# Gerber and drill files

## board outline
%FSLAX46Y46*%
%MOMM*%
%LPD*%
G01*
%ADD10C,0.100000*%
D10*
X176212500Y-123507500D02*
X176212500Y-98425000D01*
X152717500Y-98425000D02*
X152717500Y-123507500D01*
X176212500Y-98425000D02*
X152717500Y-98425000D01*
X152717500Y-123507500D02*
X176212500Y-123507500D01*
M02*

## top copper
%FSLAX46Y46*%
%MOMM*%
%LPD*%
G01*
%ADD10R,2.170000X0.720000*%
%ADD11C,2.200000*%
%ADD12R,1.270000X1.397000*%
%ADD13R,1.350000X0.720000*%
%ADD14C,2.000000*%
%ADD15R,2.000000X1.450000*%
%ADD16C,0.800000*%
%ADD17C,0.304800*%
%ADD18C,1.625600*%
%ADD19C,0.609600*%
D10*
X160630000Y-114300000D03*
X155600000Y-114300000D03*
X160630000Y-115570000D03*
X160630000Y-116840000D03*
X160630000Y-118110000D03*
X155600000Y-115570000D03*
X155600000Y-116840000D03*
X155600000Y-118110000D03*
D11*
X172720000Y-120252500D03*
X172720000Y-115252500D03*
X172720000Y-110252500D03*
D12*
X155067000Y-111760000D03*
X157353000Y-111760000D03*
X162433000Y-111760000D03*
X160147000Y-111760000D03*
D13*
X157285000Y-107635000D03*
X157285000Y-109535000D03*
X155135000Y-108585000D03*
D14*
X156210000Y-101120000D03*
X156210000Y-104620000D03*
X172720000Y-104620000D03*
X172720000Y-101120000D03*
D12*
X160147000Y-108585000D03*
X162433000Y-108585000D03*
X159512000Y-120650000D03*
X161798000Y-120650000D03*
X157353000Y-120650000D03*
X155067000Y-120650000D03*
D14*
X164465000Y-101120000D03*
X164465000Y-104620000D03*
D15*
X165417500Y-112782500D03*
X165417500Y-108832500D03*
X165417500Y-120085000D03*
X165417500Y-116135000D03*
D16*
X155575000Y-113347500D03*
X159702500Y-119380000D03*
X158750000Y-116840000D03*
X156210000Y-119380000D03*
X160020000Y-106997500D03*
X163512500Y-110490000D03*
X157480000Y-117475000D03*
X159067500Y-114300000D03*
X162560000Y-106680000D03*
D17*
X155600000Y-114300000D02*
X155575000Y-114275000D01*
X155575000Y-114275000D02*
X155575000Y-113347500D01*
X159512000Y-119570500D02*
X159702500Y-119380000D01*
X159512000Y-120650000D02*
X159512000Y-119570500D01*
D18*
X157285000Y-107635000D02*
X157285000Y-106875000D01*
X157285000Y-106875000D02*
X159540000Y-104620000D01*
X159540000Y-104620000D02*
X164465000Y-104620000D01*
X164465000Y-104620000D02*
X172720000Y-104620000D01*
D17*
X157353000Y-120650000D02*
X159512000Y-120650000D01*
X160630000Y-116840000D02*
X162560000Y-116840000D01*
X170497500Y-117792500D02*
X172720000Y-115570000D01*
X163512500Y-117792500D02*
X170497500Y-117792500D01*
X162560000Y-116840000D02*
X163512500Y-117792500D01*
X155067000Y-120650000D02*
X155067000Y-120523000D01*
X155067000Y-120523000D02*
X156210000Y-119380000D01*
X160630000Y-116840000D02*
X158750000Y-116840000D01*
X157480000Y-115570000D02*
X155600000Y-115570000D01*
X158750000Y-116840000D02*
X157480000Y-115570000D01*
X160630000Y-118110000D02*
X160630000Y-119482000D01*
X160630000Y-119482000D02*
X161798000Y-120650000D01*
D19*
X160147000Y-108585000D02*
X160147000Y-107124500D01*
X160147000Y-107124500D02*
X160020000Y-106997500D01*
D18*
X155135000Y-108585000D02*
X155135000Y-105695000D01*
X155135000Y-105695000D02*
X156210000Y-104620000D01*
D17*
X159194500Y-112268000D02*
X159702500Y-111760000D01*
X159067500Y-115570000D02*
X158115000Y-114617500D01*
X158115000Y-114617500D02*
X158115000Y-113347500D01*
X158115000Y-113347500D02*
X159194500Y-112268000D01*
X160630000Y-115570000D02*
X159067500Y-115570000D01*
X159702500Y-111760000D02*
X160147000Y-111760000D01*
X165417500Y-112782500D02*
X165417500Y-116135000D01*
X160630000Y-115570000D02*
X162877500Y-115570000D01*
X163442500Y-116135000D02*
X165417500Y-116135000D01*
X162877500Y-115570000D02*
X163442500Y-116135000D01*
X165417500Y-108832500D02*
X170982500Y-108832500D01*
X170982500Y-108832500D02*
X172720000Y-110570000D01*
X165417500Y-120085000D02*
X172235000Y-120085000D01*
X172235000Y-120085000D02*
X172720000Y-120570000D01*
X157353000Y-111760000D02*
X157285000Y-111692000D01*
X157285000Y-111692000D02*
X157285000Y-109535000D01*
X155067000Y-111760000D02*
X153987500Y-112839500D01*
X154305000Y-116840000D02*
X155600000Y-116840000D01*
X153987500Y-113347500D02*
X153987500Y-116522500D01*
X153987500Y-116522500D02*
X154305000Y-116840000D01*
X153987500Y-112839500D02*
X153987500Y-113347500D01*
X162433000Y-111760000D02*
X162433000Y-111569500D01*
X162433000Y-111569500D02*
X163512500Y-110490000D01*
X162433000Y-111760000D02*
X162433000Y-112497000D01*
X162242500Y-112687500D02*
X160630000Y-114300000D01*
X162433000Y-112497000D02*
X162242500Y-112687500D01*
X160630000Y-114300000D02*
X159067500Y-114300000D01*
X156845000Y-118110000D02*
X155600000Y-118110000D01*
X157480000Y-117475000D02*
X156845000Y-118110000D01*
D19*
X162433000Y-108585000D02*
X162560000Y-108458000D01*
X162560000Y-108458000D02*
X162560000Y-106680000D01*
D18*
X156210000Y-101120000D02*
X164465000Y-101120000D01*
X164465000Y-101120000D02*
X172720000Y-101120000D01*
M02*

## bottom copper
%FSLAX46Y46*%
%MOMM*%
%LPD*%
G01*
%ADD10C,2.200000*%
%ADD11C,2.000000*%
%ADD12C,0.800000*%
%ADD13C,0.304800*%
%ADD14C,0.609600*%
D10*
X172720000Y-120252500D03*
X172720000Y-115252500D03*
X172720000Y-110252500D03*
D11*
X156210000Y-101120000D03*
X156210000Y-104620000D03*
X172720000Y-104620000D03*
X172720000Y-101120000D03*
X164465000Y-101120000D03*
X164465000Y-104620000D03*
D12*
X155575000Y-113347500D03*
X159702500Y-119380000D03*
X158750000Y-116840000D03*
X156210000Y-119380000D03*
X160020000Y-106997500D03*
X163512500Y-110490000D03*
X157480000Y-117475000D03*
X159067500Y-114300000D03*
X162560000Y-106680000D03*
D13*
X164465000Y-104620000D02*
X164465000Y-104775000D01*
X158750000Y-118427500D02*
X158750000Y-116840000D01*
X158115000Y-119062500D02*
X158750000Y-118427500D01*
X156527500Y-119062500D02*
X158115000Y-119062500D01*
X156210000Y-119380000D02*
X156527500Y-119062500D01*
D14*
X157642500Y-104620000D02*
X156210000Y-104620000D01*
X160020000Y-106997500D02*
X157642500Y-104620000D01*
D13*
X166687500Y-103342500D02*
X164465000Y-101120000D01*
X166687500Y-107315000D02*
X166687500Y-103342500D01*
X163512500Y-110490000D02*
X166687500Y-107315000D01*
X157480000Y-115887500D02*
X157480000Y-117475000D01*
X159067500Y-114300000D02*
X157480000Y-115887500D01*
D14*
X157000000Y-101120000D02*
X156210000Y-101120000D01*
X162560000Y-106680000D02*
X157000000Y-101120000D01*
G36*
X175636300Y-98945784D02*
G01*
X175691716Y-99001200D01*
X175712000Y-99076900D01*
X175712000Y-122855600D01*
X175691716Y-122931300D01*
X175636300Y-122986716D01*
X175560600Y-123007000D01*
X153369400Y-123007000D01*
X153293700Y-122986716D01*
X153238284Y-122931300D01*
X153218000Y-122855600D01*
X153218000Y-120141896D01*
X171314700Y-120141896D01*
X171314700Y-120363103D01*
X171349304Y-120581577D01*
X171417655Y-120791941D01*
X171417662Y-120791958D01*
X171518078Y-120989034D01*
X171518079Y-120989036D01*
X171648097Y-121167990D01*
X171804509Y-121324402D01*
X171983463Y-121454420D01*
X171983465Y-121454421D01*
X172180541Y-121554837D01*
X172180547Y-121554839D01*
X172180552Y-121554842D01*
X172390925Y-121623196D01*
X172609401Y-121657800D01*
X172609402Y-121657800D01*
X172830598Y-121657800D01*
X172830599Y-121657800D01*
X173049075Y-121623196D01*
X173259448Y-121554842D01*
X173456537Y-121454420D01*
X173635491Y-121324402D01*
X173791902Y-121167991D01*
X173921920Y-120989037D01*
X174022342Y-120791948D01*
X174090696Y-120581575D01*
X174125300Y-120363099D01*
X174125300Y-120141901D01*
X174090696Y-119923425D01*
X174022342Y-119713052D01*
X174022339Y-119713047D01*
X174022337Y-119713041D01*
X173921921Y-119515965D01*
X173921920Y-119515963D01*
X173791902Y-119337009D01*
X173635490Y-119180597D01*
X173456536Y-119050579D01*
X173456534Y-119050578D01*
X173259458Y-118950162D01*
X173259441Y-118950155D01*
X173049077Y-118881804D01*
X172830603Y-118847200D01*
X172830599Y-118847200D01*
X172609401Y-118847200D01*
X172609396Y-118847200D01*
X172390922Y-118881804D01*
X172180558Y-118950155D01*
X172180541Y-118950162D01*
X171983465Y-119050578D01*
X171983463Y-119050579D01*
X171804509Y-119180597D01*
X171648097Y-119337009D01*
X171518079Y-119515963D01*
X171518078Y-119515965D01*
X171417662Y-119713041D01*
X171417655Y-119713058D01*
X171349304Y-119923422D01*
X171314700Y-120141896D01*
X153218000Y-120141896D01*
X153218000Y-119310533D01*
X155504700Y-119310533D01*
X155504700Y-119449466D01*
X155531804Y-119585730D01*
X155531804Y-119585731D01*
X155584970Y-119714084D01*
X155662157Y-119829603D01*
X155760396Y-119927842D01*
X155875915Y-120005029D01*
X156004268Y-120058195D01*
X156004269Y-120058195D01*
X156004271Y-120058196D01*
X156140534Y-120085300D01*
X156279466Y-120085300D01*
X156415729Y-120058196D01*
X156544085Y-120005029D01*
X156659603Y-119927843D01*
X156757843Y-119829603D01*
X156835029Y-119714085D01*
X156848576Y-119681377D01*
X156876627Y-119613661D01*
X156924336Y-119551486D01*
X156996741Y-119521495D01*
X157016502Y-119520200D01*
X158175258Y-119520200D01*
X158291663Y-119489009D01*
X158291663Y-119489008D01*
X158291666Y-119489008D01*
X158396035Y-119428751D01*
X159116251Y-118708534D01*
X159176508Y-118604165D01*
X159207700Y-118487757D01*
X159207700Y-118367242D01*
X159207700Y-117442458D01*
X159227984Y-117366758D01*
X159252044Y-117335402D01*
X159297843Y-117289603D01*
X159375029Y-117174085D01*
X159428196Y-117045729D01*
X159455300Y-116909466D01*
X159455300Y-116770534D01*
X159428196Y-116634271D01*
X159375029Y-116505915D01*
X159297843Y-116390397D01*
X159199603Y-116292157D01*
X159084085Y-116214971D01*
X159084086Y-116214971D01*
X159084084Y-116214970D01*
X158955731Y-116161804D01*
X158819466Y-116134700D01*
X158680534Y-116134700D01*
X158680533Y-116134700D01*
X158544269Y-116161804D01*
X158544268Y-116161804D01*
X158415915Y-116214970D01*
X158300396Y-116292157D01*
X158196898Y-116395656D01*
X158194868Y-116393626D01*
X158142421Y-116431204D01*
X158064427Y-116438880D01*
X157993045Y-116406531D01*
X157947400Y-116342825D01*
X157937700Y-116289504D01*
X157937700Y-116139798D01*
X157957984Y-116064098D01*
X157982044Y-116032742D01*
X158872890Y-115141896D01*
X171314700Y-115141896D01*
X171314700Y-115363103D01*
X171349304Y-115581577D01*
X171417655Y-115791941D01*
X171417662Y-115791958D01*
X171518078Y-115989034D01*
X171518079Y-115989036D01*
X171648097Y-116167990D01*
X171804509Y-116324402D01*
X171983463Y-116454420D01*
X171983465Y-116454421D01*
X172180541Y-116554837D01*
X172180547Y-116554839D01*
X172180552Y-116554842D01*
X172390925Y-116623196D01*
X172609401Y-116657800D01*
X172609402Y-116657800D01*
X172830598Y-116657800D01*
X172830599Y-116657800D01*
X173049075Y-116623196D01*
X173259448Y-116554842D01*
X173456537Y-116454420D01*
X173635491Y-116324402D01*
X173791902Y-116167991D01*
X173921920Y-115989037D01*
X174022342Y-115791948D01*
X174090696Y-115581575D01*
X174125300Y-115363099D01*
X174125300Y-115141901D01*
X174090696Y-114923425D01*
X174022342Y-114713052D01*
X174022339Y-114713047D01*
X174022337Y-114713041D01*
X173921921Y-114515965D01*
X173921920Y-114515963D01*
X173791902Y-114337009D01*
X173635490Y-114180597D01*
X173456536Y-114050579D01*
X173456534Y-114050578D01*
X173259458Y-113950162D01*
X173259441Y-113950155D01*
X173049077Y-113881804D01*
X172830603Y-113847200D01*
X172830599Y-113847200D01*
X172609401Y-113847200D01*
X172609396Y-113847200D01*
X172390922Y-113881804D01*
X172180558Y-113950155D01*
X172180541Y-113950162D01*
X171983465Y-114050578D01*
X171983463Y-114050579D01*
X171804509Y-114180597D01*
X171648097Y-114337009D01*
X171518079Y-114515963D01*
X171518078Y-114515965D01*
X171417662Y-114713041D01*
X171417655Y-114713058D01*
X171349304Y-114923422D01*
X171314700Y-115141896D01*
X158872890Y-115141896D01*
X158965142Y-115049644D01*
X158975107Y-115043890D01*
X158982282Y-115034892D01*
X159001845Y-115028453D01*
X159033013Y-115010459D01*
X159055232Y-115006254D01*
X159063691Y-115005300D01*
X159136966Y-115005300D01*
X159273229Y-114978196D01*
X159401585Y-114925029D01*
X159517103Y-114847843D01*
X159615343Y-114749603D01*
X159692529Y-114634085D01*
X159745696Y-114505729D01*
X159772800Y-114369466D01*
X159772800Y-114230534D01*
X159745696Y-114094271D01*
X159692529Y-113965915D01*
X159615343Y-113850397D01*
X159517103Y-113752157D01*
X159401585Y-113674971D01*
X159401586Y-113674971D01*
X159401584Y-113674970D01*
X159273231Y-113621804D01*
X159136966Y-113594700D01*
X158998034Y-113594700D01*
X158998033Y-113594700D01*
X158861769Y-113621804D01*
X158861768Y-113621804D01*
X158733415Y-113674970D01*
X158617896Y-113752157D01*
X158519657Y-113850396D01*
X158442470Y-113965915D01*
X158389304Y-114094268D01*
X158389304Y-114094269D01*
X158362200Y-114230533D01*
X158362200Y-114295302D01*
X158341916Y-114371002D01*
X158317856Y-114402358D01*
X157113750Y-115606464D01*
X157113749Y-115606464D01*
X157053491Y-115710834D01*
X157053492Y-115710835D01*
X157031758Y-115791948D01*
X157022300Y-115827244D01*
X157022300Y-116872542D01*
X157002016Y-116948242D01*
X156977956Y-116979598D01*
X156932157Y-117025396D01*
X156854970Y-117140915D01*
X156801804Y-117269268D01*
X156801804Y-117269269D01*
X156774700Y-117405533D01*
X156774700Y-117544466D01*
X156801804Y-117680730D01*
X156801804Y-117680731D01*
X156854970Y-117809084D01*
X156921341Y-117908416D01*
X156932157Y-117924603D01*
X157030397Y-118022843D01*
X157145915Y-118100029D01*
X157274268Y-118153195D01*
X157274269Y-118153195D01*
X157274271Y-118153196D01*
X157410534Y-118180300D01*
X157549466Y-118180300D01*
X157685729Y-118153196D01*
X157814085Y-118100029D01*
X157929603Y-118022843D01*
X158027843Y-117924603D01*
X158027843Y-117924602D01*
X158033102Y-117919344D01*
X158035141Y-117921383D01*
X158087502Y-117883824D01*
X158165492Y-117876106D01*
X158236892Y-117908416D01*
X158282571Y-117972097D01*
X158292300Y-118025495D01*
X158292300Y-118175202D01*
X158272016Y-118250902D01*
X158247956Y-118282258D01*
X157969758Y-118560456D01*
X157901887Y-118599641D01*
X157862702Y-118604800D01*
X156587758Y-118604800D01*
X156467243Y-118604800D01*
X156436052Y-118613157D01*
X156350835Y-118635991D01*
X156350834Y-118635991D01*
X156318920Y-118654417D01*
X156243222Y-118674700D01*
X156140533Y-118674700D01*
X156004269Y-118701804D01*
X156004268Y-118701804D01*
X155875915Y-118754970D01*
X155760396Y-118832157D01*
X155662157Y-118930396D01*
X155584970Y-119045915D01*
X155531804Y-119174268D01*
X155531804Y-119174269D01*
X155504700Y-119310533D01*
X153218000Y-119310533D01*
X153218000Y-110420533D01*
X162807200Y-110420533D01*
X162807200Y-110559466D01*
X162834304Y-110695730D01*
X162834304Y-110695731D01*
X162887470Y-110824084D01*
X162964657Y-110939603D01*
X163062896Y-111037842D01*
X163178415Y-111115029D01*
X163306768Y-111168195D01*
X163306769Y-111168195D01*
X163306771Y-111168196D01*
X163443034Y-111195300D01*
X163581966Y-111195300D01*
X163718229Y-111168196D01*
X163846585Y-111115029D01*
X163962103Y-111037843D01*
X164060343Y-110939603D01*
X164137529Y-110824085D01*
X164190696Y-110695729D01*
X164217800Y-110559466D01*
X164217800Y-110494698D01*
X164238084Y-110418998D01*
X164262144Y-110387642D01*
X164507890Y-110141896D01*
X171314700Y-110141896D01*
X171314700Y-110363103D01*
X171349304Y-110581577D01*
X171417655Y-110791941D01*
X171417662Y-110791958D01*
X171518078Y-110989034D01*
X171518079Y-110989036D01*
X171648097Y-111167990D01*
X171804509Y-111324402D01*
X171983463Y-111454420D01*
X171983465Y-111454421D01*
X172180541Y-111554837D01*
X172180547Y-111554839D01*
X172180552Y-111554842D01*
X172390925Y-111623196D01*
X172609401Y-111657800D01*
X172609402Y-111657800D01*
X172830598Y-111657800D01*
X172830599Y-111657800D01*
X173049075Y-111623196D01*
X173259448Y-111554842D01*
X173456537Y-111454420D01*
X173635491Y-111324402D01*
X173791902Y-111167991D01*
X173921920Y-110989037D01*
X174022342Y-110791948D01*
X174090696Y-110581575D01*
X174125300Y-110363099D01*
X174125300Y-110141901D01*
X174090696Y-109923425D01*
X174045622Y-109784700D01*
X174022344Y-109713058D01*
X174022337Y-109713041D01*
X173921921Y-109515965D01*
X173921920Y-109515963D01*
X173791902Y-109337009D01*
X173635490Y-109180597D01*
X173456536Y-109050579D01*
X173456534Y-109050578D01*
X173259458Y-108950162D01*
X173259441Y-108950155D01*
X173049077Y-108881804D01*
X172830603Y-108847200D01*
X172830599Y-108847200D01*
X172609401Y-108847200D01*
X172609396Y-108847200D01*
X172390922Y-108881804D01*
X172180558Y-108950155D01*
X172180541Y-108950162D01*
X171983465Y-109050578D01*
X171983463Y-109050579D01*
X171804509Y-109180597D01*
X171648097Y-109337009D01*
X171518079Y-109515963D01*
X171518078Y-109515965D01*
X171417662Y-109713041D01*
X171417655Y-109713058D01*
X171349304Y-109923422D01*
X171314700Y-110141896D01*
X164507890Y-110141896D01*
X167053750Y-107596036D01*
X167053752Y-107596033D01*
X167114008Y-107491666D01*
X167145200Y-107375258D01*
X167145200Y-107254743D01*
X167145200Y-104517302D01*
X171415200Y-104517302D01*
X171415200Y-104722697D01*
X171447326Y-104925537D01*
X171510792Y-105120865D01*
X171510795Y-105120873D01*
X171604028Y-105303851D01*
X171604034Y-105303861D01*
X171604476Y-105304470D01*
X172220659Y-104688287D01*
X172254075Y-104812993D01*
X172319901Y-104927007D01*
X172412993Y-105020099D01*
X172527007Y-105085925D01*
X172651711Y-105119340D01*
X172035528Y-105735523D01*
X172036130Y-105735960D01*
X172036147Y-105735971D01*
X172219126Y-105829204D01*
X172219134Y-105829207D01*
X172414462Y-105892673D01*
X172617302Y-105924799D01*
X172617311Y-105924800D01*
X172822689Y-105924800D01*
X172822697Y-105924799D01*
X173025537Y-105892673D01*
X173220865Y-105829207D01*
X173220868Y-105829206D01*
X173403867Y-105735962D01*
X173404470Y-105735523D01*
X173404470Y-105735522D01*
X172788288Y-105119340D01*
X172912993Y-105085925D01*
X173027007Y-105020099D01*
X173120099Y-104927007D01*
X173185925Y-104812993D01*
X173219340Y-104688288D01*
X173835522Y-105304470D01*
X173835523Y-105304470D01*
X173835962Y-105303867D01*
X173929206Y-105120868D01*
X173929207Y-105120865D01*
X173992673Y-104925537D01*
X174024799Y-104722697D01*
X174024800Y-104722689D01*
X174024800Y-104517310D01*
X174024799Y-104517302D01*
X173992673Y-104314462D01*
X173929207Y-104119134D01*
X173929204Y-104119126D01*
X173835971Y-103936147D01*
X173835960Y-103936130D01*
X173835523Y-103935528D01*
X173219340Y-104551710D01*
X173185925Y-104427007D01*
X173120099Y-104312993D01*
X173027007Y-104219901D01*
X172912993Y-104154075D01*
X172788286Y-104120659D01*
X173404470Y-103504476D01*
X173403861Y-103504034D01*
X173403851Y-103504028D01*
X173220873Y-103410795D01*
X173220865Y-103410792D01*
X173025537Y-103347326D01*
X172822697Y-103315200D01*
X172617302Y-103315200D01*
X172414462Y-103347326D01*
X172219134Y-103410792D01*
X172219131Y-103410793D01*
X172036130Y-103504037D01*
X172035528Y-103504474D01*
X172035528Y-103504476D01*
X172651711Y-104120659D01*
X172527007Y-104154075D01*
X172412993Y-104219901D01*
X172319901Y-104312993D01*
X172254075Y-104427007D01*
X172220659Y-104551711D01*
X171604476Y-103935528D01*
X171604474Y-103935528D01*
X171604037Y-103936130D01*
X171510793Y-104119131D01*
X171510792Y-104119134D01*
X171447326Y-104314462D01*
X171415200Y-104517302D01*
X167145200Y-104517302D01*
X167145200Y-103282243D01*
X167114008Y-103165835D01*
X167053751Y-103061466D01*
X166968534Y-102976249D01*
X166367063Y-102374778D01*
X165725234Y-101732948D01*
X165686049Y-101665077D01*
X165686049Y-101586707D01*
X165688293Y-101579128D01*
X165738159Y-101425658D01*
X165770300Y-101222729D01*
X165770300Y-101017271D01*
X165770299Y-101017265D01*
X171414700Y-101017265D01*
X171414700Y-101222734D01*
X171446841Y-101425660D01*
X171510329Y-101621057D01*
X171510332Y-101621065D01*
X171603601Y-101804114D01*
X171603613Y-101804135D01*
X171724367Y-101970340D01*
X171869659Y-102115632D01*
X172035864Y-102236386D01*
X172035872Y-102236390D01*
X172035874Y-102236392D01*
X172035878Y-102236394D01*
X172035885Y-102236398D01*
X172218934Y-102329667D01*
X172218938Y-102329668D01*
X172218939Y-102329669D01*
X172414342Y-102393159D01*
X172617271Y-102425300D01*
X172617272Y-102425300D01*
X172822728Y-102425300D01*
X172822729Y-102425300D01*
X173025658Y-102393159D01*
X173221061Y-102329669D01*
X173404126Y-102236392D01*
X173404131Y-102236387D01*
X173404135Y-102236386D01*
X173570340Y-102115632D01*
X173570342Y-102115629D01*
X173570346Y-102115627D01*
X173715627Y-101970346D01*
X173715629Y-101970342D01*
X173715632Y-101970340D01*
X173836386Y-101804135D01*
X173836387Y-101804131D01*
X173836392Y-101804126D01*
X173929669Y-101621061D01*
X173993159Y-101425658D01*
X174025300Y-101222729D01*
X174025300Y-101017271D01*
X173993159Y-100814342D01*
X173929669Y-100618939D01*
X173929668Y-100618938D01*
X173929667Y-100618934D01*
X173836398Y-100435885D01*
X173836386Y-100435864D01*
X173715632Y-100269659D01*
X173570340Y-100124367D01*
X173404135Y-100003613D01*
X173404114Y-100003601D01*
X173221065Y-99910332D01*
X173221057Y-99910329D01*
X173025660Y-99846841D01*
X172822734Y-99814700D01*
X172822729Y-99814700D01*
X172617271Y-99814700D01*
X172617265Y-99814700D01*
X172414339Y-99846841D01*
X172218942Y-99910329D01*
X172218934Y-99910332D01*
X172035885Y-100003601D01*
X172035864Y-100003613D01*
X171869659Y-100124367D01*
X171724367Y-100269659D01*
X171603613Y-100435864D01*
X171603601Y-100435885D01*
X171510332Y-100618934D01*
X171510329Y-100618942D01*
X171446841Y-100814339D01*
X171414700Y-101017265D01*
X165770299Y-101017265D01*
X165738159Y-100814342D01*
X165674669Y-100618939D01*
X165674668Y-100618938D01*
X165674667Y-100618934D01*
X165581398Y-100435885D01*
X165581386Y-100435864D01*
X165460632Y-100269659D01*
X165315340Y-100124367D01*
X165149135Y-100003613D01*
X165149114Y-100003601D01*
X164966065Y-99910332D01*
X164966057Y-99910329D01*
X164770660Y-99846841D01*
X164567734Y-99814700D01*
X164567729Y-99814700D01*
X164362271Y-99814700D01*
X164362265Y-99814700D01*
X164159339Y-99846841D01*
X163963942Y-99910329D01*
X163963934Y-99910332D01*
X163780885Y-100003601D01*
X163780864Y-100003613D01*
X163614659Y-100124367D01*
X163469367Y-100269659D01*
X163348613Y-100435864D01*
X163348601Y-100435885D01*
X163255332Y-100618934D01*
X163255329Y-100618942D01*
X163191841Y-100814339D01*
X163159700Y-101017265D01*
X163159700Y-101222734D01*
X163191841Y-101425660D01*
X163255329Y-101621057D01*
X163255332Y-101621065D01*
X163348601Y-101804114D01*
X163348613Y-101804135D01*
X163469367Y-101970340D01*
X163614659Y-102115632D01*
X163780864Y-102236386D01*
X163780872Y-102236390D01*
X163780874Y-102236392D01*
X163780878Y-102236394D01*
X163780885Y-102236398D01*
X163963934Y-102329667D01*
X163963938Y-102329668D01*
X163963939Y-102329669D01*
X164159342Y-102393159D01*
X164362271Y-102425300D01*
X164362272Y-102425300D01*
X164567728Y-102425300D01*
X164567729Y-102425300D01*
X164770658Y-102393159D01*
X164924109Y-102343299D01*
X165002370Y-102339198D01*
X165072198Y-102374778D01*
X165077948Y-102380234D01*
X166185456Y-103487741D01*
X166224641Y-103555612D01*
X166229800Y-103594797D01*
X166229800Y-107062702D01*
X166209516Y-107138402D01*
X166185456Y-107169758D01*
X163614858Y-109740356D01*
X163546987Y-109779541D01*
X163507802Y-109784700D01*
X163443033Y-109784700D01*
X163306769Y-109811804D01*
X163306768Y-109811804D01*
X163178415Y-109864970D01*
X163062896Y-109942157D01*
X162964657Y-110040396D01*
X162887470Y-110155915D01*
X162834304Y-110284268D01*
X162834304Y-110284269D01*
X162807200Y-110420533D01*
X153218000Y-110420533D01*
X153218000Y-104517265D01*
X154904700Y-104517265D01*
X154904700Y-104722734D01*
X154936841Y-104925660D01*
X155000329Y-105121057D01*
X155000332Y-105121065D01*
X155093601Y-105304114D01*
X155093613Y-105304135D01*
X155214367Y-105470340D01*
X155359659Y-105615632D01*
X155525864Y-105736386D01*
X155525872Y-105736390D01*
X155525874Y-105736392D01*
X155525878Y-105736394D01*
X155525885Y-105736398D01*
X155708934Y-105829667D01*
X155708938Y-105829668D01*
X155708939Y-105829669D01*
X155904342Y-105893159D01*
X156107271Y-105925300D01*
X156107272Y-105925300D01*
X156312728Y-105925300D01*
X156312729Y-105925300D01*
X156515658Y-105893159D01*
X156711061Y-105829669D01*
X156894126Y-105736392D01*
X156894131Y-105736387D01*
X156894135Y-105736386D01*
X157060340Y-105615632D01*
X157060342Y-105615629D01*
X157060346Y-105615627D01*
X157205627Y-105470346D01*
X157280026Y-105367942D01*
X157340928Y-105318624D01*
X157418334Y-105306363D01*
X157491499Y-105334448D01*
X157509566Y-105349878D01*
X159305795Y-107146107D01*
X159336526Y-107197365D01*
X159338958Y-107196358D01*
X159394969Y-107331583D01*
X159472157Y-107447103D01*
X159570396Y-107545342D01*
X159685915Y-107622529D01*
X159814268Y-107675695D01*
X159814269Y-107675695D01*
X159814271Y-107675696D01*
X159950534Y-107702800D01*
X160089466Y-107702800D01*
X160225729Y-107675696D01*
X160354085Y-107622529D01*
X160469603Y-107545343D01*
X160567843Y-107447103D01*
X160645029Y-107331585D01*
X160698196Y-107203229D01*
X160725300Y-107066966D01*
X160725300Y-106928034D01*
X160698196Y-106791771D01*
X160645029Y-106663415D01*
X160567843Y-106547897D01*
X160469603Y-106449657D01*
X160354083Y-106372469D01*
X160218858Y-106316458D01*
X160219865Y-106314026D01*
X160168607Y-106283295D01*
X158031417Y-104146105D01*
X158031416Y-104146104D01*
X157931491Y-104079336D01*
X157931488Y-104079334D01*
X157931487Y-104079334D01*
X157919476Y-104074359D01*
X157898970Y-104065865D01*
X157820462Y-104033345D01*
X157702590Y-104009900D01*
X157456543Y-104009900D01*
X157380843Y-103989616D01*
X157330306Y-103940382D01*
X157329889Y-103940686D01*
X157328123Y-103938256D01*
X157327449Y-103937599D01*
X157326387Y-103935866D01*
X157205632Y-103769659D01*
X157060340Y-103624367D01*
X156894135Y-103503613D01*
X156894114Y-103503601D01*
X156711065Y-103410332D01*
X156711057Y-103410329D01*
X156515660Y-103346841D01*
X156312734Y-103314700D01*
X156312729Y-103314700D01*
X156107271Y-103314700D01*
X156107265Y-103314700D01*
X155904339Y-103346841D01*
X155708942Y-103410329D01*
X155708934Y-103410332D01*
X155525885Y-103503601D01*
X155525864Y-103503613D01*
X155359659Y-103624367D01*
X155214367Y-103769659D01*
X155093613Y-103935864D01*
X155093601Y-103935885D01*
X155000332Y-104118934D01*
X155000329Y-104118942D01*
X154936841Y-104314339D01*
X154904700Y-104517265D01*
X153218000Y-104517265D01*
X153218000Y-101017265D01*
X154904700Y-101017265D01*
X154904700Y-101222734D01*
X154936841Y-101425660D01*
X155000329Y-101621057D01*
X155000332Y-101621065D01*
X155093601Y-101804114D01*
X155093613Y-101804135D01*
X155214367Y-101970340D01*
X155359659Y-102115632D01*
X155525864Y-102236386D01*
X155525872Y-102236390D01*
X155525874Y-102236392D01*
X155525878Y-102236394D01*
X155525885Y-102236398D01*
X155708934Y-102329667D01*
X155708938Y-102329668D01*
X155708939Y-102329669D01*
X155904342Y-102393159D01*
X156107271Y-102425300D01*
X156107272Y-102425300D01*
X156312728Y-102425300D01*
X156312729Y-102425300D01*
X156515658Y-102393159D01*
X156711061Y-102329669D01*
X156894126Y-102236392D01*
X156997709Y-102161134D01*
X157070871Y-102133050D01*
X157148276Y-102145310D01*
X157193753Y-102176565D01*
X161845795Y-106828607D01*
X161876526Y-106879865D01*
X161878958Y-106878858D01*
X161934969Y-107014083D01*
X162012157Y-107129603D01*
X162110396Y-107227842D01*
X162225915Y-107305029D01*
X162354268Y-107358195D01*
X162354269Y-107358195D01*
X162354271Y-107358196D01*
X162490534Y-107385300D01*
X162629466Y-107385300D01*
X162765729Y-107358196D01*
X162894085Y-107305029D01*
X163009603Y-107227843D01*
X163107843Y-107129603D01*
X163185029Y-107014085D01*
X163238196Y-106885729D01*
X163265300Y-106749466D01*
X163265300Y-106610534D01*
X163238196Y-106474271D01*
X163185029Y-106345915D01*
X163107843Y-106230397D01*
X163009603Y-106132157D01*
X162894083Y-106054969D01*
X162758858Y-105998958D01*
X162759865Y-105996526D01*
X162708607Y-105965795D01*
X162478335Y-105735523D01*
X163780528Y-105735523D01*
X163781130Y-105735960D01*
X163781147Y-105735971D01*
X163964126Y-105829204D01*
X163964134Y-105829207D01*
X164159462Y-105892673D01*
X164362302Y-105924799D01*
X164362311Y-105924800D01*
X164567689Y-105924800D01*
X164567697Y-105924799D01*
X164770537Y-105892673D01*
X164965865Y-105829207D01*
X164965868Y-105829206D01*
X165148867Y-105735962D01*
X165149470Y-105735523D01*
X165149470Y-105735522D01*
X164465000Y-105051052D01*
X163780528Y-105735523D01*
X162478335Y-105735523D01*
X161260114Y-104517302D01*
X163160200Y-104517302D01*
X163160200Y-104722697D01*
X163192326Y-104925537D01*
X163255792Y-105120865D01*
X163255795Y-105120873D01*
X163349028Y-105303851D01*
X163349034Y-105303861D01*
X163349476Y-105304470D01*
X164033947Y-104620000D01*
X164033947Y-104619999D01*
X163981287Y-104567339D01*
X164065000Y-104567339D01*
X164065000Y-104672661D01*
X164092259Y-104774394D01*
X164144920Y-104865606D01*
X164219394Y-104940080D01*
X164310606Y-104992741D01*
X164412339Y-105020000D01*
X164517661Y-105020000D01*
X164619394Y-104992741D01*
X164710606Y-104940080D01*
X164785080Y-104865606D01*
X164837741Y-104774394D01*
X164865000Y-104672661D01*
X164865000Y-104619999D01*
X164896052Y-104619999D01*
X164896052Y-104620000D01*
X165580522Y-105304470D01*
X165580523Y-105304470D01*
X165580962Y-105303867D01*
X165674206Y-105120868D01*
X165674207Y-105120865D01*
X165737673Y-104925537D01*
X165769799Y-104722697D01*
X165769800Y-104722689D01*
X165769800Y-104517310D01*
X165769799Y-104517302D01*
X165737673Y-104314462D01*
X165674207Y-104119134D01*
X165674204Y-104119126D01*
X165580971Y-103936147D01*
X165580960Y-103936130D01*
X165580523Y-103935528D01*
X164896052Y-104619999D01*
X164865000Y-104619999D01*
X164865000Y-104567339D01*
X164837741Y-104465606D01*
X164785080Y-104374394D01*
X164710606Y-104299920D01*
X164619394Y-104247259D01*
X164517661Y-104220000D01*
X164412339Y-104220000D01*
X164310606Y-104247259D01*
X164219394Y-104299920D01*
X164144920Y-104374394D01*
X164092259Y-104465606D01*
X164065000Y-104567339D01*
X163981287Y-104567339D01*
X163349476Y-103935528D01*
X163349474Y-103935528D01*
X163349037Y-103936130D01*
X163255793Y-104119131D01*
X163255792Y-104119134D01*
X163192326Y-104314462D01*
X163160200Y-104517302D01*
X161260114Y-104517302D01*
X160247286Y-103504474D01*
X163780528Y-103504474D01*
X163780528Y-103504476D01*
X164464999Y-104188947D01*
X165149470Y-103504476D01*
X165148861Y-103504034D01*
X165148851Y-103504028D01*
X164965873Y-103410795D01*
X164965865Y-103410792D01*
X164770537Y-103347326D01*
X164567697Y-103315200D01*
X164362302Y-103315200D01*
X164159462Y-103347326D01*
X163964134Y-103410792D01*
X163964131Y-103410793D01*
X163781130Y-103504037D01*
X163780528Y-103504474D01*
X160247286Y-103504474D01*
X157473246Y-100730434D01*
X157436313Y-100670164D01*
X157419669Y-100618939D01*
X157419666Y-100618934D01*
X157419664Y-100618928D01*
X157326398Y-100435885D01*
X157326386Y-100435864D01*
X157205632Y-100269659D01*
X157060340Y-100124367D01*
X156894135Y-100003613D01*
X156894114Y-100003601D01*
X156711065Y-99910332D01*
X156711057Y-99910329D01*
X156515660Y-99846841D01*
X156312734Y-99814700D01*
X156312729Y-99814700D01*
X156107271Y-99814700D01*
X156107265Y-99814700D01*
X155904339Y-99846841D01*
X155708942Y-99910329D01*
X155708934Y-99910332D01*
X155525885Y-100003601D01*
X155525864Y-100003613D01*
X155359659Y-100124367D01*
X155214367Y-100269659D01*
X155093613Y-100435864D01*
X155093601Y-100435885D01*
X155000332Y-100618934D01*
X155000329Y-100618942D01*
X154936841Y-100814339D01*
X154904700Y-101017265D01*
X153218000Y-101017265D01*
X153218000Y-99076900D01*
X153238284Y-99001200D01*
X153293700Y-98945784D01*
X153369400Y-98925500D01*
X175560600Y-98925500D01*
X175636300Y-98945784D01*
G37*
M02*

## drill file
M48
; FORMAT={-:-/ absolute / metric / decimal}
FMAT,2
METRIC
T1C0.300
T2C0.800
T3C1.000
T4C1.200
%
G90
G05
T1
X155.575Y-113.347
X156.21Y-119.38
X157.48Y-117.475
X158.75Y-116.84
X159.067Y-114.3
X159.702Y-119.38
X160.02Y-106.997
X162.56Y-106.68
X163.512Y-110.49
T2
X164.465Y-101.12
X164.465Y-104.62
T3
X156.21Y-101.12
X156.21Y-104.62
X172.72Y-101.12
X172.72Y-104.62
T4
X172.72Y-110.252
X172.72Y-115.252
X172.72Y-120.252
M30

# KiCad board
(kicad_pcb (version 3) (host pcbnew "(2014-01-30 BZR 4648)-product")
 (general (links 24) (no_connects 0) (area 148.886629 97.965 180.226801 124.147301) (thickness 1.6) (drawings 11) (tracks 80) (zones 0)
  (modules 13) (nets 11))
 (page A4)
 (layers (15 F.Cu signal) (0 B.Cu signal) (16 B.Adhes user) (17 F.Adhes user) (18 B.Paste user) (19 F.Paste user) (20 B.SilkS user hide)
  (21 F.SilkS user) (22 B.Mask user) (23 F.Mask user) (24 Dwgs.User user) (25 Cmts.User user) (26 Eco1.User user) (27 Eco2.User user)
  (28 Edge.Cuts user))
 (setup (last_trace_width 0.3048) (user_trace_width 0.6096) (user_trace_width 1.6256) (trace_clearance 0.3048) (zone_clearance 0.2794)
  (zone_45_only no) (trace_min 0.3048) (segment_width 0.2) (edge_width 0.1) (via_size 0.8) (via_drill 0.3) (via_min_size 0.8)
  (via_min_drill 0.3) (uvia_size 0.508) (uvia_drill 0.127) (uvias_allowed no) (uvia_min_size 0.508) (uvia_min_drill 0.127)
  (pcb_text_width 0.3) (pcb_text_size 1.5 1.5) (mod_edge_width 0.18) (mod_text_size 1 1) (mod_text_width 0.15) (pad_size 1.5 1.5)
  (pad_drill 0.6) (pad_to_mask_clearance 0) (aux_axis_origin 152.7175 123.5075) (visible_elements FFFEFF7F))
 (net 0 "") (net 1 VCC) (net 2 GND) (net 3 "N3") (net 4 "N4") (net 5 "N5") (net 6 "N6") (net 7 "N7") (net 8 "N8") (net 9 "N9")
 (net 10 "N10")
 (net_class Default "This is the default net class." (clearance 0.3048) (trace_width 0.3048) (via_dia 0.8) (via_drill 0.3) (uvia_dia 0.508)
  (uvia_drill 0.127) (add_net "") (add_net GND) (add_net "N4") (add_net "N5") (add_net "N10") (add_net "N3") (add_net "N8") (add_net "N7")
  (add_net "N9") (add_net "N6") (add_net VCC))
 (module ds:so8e (layer F.Cu) (at 158.115 116.205 270)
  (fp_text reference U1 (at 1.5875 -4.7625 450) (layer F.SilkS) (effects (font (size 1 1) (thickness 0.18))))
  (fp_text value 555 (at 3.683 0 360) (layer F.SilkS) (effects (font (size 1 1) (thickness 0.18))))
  (pad 8 smd rect (at -1.905 -2.515 270) (size 0.72 2.17) (layers F.Cu F.Paste F.Mask) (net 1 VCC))
  (pad 1 smd rect (at -1.905 2.515 270) (size 0.72 2.17) (layers F.Cu F.Paste F.Mask) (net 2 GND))
  (pad 7 smd rect (at -0.635 -2.515 270) (size 0.72 2.17) (layers F.Cu F.Paste F.Mask) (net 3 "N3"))
  (pad 6 smd rect (at 0.635 -2.515 270) (size 0.72 2.17) (layers F.Cu F.Paste F.Mask) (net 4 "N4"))
  (pad 5 smd rect (at 1.905 -2.515 270) (size 0.72 2.17) (layers F.Cu F.Paste F.Mask) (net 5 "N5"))
  (pad 2 smd rect (at -0.635 2.515 270) (size 0.72 2.17) (layers F.Cu F.Paste F.Mask) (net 4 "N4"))
  (pad 3 smd rect (at 0.635 2.515 270) (size 0.72 2.17) (layers F.Cu F.Paste F.Mask) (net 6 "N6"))
  (pad 4 smd rect (at 1.905 2.515 270) (size 0.72 2.17) (layers F.Cu F.Paste F.Mask) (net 1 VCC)))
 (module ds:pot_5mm (layer F.Cu) (at 172.72 115.2525 90)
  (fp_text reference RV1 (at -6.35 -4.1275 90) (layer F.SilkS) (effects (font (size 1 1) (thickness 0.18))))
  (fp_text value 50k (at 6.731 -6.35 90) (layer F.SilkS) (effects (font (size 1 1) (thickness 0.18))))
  (pad 1 thru_hole circle (at -5 0 90) (size 2.2 2.2) (drill 1.2) (layers *.Cu *.Mask F.SilkS) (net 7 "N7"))
  (pad 2 thru_hole circle (at 0 0 90) (size 2.2 2.2) (drill 1.2) (layers *.Cu *.Mask F.SilkS) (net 4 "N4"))
  (pad 3 thru_hole circle (at 5 0 90) (size 2.2 2.2) (drill 1.2) (layers *.Cu *.Mask F.SilkS) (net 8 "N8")))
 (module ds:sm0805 (layer F.Cu) (at 156.21 111.76)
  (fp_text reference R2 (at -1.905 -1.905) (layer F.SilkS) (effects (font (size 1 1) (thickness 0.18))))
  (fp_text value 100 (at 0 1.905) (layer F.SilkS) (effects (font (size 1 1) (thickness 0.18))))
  (pad 1 smd rect (at -1.143 0) (size 1.27 1.397) (layers F.Cu F.Paste F.Mask) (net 6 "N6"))
  (pad 2 smd rect (at 1.143 0) (size 1.27 1.397) (layers F.Cu F.Paste F.Mask) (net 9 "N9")))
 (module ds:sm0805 (layer F.Cu) (at 161.29 111.76 180)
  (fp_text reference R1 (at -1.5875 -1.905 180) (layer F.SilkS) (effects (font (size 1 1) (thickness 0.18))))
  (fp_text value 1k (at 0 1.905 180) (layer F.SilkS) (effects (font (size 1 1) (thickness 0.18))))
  (pad 1 smd rect (at -1.143 0 180) (size 1.27 1.397) (layers F.Cu F.Paste F.Mask) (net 1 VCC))
  (pad 2 smd rect (at 1.143 0 180) (size 1.27 1.397) (layers F.Cu F.Paste F.Mask) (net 3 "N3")))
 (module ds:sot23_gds (layer F.Cu) (at 156.21 108.585 270)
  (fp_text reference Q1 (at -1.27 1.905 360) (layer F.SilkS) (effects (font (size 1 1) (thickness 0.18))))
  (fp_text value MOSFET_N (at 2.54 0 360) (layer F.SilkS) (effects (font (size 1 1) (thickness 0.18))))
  (pad S smd rect (at -0.95 -1.075 270) (size 0.72 1.35) (layers F.Cu F.Paste F.Mask) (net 2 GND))
  (pad G smd rect (at 0.95 -1.075 270) (size 0.72 1.35) (layers F.Cu F.Paste F.Mask) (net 9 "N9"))
  (pad D smd rect (at 0 1.075 270) (size 0.72 1.35) (layers F.Cu F.Paste F.Mask) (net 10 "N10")))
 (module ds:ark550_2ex (layer F.Cu) (at 156.21 102.87 270)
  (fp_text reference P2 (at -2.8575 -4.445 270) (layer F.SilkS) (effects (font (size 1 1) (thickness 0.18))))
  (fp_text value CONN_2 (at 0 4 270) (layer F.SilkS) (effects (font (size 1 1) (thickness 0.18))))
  (pad 1 thru_hole circle (at -1.75 0 270) (size 2 2) (drill 1) (layers *.Cu *.Mask F.SilkS) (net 1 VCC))
  (pad 2 thru_hole circle (at 1.75 0 270) (size 2 2) (drill 1) (layers *.Cu *.Mask F.SilkS) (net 10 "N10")))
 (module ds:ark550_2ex (layer F.Cu) (at 172.72 102.87 90)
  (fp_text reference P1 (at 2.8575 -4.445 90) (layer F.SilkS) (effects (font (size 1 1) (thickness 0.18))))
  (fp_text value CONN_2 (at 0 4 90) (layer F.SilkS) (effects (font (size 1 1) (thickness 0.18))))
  (pad 1 thru_hole circle (at -1.75 0 90) (size 2 2) (drill 1) (layers *.Cu *.Mask F.SilkS) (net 2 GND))
  (pad 2 thru_hole circle (at 1.75 0 90) (size 2 2) (drill 1) (layers *.Cu *.Mask F.SilkS) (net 1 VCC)))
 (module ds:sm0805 (layer F.Cu) (at 161.29 108.585)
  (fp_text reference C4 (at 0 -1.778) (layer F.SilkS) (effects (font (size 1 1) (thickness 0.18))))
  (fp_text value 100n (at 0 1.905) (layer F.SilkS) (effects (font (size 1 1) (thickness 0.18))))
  (pad 1 smd rect (at -1.143 0) (size 1.27 1.397) (layers F.Cu F.Paste F.Mask) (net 10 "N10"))
  (pad 2 smd rect (at 1.143 0) (size 1.27 1.397) (layers F.Cu F.Paste F.Mask) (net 1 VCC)))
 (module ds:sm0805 (layer F.Cu) (at 160.655 120.65)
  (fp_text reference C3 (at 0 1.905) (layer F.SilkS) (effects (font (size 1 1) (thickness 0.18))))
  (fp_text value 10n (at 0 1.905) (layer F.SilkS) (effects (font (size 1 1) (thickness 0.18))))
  (pad 1 smd rect (at -1.143 0) (size 1.27 1.397) (layers F.Cu F.Paste F.Mask) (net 2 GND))
  (pad 2 smd rect (at 1.143 0) (size 1.27 1.397) (layers F.Cu F.Paste F.Mask) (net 5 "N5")))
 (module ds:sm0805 (layer F.Cu) (at 156.21 120.65 180)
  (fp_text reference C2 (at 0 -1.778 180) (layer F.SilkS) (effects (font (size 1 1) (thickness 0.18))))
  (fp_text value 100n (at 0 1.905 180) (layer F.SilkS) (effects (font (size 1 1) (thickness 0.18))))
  (pad 1 smd rect (at -1.143 0 180) (size 1.27 1.397) (layers F.Cu F.Paste F.Mask) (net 2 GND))
  (pad 2 smd rect (at 1.143 0 180) (size 1.27 1.397) (layers F.Cu F.Paste F.Mask) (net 4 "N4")))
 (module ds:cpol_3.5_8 (layer F.Cu) (at 164.465 102.87 270)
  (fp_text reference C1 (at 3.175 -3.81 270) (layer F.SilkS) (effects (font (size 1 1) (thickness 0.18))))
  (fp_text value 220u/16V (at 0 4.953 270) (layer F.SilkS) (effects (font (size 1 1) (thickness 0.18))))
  (pad 1 thru_hole circle (at -1.75 0 270) (size 2 2) (drill 0.8) (layers *.Cu *.Mask F.SilkS) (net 1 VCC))
  (pad 2 thru_hole circle (at 1.75 0 270) (size 2 2) (drill 0.8) (layers *.Cu *.Mask F.SilkS) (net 2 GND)))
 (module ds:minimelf (layer F.Cu) (at 165.4175 110.8075 90)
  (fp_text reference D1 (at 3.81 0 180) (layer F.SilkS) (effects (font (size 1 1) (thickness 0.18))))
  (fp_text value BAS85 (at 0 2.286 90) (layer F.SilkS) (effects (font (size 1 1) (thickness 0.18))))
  (pad 1 smd rect (at -1.975 0 90) (size 1.45 2) (layers F.Cu F.Paste F.Mask) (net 3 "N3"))
  (pad 2 smd rect (at 1.975 0 90) (size 1.45 2) (layers F.Cu F.Paste F.Mask) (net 8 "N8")))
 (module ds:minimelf (layer F.Cu) (at 165.4175 118.11 90)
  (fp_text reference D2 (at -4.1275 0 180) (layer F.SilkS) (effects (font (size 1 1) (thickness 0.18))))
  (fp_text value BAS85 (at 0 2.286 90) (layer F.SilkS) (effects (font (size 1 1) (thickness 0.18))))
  (pad 1 smd rect (at -1.975 0 90) (size 1.45 2) (layers F.Cu F.Paste F.Mask) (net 7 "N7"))
  (pad 2 smd rect (at 1.975 0 90) (size 1.45 2) (layers F.Cu F.Paste F.Mask) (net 3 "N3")))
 (gr_line (start 176.2125 123.5075) (end 176.2125 98.425) (angle 90) (layer Edge.Cuts) (width 0.1))
 (gr_line (start 152.7175 98.425) (end 152.7175 123.5075) (angle 90) (layer Edge.Cuts) (width 0.1))
 (gr_line (start 176.2125 98.425) (end 152.7175 98.425) (angle 90) (layer Edge.Cuts) (width 0.1))
 (gr_line (start 152.7175 123.5075) (end 176.2125 123.5075) (angle 90) (layer Edge.Cuts) (width 0.1))
 (segment (start 164.465 104.62) (end 164.465 104.775) (width 0.3048) (layer B.Cu) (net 2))
 (segment (start 155.6 114.3) (end 155.575 114.275) (width 0.3048) (layer F.Cu) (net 2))
 (segment (start 155.575 114.275) (end 155.575 113.3475) (width 0.3048) (layer F.Cu) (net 2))
 (via (at 155.575 113.3475) (size 0.8) (layers F.Cu B.Cu) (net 2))
 (segment (start 159.512 119.5705) (end 159.7025 119.38) (width 0.3048) (layer F.Cu) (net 2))
 (segment (start 159.512 120.65) (end 159.512 119.5705) (width 0.3048) (layer F.Cu) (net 2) (status 10))
 (via (at 159.7025 119.38) (size 0.8) (layers F.Cu B.Cu) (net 2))
 (segment (start 157.285 107.635) (end 157.285 106.875) (width 1.6256) (layer F.Cu) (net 2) (status 10))
 (segment (start 157.285 106.875) (end 159.54 104.62) (width 1.6256) (layer F.Cu) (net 2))
 (segment (start 159.54 104.62) (end 164.465 104.62) (width 1.6256) (layer F.Cu) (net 2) (status 20))
 (segment (start 164.465 104.62) (end 172.72 104.62) (width 1.6256) (layer F.Cu) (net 2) (status 30))
 (segment (start 157.353 120.65) (end 159.512 120.65) (width 0.3048) (layer F.Cu) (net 2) (status 30))
 (segment (start 160.63 116.84) (end 162.56 116.84) (width 0.3048) (layer F.Cu) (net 4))
 (segment (start 170.4975 117.7925) (end 172.72 115.57) (width 0.3048) (layer F.Cu) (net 4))
 (segment (start 163.5125 117.7925) (end 170.4975 117.7925) (width 0.3048) (layer F.Cu) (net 4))
 (segment (start 162.56 116.84) (end 163.5125 117.7925) (width 0.3048) (layer F.Cu) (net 4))
 (segment (start 155.067 120.65) (end 155.067 120.523) (width 0.3048) (layer F.Cu) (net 4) (status 30))
 (via (at 158.75 116.84) (size 0.8) (layers F.Cu B.Cu) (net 4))
 (segment (start 158.75 118.4275) (end 158.75 116.84) (width 0.3048) (layer B.Cu) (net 4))
 (segment (start 158.115 119.0625) (end 158.75 118.4275) (width 0.3048) (layer B.Cu) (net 4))
 (segment (start 156.5275 119.0625) (end 158.115 119.0625) (width 0.3048) (layer B.Cu) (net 4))
 (segment (start 156.21 119.38) (end 156.5275 119.0625) (width 0.3048) (layer B.Cu) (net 4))
 (via (at 156.21 119.38) (size 0.8) (layers F.Cu B.Cu) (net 4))
 (segment (start 155.067 120.523) (end 156.21 119.38) (width 0.3048) (layer F.Cu) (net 4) (status 10))
 (segment (start 160.63 116.84) (end 158.75 116.84) (width 0.3048) (layer F.Cu) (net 4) (status 10))
 (segment (start 157.48 115.57) (end 155.6 115.57) (width 0.3048) (layer F.Cu) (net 4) (status 20))
 (segment (start 158.75 116.84) (end 157.48 115.57) (width 0.3048) (layer F.Cu) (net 4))
 (segment (start 160.63 118.11) (end 160.63 119.482) (width 0.3048) (layer F.Cu) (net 5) (status 10))
 (segment (start 160.63 119.482) (end 161.798 120.65) (width 0.3048) (layer F.Cu) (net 5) (status 20))
 (segment (start 160.147 108.585) (end 160.147 107.1245) (width 0.6096) (layer F.Cu) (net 10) (status 10))
 (segment (start 157.6425 104.62) (end 156.21 104.62) (width 0.6096) (layer B.Cu) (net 10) (status 20))
 (segment (start 160.02 106.9975) (end 157.6425 104.62) (width 0.6096) (layer B.Cu) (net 10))
 (via (at 160.02 106.9975) (size 0.8) (layers F.Cu B.Cu) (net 10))
 (segment (start 160.147 107.1245) (end 160.02 106.9975) (width 0.6096) (layer F.Cu) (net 10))
 (segment (start 155.135 108.585) (end 155.135 105.695) (width 1.6256) (layer F.Cu) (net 10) (status 10))
 (segment (start 155.135 105.695) (end 156.21 104.62) (width 1.6256) (layer F.Cu) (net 10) (status 20))
 (segment (start 159.1945 112.268) (end 159.7025 111.76) (width 0.3048) (layer F.Cu) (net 3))
 (segment (start 159.0675 115.57) (end 158.115 114.6175) (width 0.3048) (layer F.Cu) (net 3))
 (segment (start 158.115 114.6175) (end 158.115 113.3475) (width 0.3048) (layer F.Cu) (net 3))
 (segment (start 158.115 113.3475) (end 159.1945 112.268) (width 0.3048) (layer F.Cu) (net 3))
 (segment (start 160.63 115.57) (end 159.0675 115.57) (width 0.3048) (layer F.Cu) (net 3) (status 10))
 (segment (start 159.7025 111.76) (end 160.147 111.76) (width 0.3048) (layer F.Cu) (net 3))
 (segment (start 165.4175 112.7825) (end 165.4175 116.135) (width 0.3048) (layer F.Cu) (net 3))
 (segment (start 160.63 115.57) (end 162.8775 115.57) (width 0.3048) (layer F.Cu) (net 3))
 (segment (start 163.4425 116.135) (end 165.4175 116.135) (width 0.3048) (layer F.Cu) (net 3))
 (segment (start 162.8775 115.57) (end 163.4425 116.135) (width 0.3048) (layer F.Cu) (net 3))
 (segment (start 165.4175 108.8325) (end 170.9825 108.8325) (width 0.3048) (layer F.Cu) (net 8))
 (segment (start 170.9825 108.8325) (end 172.72 110.57) (width 0.3048) (layer F.Cu) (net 8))
 (segment (start 165.4175 120.085) (end 172.235 120.085) (width 0.3048) (layer F.Cu) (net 7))
 (segment (start 172.235 120.085) (end 172.72 120.57) (width 0.3048) (layer F.Cu) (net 7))
 (segment (start 157.353 111.76) (end 157.285 111.692) (width 0.3048) (layer F.Cu) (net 9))
 (segment (start 157.285 111.692) (end 157.285 109.535) (width 0.3048) (layer F.Cu) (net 9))
 (segment (start 155.067 111.76) (end 153.9875 112.8395) (width 0.3048) (layer F.Cu) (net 6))
 (segment (start 154.305 116.84) (end 155.6 116.84) (width 0.3048) (layer F.Cu) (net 6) (status 20))
 (segment (start 153.9875 113.3475) (end 153.9875 116.5225) (width 0.3048) (layer F.Cu) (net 6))
 (segment (start 153.9875 116.5225) (end 154.305 116.84) (width 0.3048) (layer F.Cu) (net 6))
 (segment (start 153.9875 112.8395) (end 153.9875 113.3475) (width 0.3048) (layer F.Cu) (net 6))
 (segment (start 162.433 111.76) (end 162.433 111.5695) (width 0.3048) (layer F.Cu) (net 1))
 (segment (start 166.6875 103.3425) (end 164.465 101.12) (width 0.3048) (layer B.Cu) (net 1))
 (segment (start 166.6875 107.315) (end 166.6875 103.3425) (width 0.3048) (layer B.Cu) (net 1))
 (segment (start 163.5125 110.49) (end 166.6875 107.315) (width 0.3048) (layer B.Cu) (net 1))
 (via (at 163.5125 110.49) (size 0.8) (layers F.Cu B.Cu) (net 1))
 (segment (start 162.433 111.5695) (end 163.5125 110.49) (width 0.3048) (layer F.Cu) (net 1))
 (segment (start 162.433 111.76) (end 162.433 112.497) (width 0.3048) (layer F.Cu) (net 1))
 (segment (start 162.2425 112.6875) (end 160.63 114.3) (width 0.3048) (layer F.Cu) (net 1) (status 20))
 (segment (start 162.433 112.497) (end 162.2425 112.6875) (width 0.3048) (layer F.Cu) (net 1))
 (segment (start 160.63 114.3) (end 159.0675 114.3) (width 0.3048) (layer F.Cu) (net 1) (status 10))
 (segment (start 156.845 118.11) (end 155.6 118.11) (width 0.3048) (layer F.Cu) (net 1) (status 20))
 (segment (start 157.48 117.475) (end 156.845 118.11) (width 0.3048) (layer F.Cu) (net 1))
 (via (at 157.48 117.475) (size 0.8) (layers F.Cu B.Cu) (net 1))
 (segment (start 157.48 115.8875) (end 157.48 117.475) (width 0.3048) (layer B.Cu) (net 1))
 (segment (start 159.0675 114.3) (end 157.48 115.8875) (width 0.3048) (layer B.Cu) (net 1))
 (via (at 159.0675 114.3) (size 0.8) (layers F.Cu B.Cu) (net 1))
 (segment (start 162.433 108.585) (end 162.56 108.458) (width 0.6096) (layer F.Cu) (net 1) (status 30))
 (segment (start 162.56 108.458) (end 162.56 106.68) (width 0.6096) (layer F.Cu) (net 1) (status 10))
 (segment (start 157 101.12) (end 156.21 101.12) (width 0.6096) (layer B.Cu) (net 1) (status 30))
 (segment (start 162.56 106.68) (end 157 101.12) (width 0.6096) (layer B.Cu) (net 1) (status 20))
 (via (at 162.56 106.68) (size 0.8) (layers F.Cu B.Cu) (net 1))
 (segment (start 156.21 101.12) (end 164.465 101.12) (width 1.6256) (layer F.Cu) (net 1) (status 30))
 (segment (start 164.465 101.12) (end 172.72 101.12) (width 1.6256) (layer F.Cu) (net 1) (status 30))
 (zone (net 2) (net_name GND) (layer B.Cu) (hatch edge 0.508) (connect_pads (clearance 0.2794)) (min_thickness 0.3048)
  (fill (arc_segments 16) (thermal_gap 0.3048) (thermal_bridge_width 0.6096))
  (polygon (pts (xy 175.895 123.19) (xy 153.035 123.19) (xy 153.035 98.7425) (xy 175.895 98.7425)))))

